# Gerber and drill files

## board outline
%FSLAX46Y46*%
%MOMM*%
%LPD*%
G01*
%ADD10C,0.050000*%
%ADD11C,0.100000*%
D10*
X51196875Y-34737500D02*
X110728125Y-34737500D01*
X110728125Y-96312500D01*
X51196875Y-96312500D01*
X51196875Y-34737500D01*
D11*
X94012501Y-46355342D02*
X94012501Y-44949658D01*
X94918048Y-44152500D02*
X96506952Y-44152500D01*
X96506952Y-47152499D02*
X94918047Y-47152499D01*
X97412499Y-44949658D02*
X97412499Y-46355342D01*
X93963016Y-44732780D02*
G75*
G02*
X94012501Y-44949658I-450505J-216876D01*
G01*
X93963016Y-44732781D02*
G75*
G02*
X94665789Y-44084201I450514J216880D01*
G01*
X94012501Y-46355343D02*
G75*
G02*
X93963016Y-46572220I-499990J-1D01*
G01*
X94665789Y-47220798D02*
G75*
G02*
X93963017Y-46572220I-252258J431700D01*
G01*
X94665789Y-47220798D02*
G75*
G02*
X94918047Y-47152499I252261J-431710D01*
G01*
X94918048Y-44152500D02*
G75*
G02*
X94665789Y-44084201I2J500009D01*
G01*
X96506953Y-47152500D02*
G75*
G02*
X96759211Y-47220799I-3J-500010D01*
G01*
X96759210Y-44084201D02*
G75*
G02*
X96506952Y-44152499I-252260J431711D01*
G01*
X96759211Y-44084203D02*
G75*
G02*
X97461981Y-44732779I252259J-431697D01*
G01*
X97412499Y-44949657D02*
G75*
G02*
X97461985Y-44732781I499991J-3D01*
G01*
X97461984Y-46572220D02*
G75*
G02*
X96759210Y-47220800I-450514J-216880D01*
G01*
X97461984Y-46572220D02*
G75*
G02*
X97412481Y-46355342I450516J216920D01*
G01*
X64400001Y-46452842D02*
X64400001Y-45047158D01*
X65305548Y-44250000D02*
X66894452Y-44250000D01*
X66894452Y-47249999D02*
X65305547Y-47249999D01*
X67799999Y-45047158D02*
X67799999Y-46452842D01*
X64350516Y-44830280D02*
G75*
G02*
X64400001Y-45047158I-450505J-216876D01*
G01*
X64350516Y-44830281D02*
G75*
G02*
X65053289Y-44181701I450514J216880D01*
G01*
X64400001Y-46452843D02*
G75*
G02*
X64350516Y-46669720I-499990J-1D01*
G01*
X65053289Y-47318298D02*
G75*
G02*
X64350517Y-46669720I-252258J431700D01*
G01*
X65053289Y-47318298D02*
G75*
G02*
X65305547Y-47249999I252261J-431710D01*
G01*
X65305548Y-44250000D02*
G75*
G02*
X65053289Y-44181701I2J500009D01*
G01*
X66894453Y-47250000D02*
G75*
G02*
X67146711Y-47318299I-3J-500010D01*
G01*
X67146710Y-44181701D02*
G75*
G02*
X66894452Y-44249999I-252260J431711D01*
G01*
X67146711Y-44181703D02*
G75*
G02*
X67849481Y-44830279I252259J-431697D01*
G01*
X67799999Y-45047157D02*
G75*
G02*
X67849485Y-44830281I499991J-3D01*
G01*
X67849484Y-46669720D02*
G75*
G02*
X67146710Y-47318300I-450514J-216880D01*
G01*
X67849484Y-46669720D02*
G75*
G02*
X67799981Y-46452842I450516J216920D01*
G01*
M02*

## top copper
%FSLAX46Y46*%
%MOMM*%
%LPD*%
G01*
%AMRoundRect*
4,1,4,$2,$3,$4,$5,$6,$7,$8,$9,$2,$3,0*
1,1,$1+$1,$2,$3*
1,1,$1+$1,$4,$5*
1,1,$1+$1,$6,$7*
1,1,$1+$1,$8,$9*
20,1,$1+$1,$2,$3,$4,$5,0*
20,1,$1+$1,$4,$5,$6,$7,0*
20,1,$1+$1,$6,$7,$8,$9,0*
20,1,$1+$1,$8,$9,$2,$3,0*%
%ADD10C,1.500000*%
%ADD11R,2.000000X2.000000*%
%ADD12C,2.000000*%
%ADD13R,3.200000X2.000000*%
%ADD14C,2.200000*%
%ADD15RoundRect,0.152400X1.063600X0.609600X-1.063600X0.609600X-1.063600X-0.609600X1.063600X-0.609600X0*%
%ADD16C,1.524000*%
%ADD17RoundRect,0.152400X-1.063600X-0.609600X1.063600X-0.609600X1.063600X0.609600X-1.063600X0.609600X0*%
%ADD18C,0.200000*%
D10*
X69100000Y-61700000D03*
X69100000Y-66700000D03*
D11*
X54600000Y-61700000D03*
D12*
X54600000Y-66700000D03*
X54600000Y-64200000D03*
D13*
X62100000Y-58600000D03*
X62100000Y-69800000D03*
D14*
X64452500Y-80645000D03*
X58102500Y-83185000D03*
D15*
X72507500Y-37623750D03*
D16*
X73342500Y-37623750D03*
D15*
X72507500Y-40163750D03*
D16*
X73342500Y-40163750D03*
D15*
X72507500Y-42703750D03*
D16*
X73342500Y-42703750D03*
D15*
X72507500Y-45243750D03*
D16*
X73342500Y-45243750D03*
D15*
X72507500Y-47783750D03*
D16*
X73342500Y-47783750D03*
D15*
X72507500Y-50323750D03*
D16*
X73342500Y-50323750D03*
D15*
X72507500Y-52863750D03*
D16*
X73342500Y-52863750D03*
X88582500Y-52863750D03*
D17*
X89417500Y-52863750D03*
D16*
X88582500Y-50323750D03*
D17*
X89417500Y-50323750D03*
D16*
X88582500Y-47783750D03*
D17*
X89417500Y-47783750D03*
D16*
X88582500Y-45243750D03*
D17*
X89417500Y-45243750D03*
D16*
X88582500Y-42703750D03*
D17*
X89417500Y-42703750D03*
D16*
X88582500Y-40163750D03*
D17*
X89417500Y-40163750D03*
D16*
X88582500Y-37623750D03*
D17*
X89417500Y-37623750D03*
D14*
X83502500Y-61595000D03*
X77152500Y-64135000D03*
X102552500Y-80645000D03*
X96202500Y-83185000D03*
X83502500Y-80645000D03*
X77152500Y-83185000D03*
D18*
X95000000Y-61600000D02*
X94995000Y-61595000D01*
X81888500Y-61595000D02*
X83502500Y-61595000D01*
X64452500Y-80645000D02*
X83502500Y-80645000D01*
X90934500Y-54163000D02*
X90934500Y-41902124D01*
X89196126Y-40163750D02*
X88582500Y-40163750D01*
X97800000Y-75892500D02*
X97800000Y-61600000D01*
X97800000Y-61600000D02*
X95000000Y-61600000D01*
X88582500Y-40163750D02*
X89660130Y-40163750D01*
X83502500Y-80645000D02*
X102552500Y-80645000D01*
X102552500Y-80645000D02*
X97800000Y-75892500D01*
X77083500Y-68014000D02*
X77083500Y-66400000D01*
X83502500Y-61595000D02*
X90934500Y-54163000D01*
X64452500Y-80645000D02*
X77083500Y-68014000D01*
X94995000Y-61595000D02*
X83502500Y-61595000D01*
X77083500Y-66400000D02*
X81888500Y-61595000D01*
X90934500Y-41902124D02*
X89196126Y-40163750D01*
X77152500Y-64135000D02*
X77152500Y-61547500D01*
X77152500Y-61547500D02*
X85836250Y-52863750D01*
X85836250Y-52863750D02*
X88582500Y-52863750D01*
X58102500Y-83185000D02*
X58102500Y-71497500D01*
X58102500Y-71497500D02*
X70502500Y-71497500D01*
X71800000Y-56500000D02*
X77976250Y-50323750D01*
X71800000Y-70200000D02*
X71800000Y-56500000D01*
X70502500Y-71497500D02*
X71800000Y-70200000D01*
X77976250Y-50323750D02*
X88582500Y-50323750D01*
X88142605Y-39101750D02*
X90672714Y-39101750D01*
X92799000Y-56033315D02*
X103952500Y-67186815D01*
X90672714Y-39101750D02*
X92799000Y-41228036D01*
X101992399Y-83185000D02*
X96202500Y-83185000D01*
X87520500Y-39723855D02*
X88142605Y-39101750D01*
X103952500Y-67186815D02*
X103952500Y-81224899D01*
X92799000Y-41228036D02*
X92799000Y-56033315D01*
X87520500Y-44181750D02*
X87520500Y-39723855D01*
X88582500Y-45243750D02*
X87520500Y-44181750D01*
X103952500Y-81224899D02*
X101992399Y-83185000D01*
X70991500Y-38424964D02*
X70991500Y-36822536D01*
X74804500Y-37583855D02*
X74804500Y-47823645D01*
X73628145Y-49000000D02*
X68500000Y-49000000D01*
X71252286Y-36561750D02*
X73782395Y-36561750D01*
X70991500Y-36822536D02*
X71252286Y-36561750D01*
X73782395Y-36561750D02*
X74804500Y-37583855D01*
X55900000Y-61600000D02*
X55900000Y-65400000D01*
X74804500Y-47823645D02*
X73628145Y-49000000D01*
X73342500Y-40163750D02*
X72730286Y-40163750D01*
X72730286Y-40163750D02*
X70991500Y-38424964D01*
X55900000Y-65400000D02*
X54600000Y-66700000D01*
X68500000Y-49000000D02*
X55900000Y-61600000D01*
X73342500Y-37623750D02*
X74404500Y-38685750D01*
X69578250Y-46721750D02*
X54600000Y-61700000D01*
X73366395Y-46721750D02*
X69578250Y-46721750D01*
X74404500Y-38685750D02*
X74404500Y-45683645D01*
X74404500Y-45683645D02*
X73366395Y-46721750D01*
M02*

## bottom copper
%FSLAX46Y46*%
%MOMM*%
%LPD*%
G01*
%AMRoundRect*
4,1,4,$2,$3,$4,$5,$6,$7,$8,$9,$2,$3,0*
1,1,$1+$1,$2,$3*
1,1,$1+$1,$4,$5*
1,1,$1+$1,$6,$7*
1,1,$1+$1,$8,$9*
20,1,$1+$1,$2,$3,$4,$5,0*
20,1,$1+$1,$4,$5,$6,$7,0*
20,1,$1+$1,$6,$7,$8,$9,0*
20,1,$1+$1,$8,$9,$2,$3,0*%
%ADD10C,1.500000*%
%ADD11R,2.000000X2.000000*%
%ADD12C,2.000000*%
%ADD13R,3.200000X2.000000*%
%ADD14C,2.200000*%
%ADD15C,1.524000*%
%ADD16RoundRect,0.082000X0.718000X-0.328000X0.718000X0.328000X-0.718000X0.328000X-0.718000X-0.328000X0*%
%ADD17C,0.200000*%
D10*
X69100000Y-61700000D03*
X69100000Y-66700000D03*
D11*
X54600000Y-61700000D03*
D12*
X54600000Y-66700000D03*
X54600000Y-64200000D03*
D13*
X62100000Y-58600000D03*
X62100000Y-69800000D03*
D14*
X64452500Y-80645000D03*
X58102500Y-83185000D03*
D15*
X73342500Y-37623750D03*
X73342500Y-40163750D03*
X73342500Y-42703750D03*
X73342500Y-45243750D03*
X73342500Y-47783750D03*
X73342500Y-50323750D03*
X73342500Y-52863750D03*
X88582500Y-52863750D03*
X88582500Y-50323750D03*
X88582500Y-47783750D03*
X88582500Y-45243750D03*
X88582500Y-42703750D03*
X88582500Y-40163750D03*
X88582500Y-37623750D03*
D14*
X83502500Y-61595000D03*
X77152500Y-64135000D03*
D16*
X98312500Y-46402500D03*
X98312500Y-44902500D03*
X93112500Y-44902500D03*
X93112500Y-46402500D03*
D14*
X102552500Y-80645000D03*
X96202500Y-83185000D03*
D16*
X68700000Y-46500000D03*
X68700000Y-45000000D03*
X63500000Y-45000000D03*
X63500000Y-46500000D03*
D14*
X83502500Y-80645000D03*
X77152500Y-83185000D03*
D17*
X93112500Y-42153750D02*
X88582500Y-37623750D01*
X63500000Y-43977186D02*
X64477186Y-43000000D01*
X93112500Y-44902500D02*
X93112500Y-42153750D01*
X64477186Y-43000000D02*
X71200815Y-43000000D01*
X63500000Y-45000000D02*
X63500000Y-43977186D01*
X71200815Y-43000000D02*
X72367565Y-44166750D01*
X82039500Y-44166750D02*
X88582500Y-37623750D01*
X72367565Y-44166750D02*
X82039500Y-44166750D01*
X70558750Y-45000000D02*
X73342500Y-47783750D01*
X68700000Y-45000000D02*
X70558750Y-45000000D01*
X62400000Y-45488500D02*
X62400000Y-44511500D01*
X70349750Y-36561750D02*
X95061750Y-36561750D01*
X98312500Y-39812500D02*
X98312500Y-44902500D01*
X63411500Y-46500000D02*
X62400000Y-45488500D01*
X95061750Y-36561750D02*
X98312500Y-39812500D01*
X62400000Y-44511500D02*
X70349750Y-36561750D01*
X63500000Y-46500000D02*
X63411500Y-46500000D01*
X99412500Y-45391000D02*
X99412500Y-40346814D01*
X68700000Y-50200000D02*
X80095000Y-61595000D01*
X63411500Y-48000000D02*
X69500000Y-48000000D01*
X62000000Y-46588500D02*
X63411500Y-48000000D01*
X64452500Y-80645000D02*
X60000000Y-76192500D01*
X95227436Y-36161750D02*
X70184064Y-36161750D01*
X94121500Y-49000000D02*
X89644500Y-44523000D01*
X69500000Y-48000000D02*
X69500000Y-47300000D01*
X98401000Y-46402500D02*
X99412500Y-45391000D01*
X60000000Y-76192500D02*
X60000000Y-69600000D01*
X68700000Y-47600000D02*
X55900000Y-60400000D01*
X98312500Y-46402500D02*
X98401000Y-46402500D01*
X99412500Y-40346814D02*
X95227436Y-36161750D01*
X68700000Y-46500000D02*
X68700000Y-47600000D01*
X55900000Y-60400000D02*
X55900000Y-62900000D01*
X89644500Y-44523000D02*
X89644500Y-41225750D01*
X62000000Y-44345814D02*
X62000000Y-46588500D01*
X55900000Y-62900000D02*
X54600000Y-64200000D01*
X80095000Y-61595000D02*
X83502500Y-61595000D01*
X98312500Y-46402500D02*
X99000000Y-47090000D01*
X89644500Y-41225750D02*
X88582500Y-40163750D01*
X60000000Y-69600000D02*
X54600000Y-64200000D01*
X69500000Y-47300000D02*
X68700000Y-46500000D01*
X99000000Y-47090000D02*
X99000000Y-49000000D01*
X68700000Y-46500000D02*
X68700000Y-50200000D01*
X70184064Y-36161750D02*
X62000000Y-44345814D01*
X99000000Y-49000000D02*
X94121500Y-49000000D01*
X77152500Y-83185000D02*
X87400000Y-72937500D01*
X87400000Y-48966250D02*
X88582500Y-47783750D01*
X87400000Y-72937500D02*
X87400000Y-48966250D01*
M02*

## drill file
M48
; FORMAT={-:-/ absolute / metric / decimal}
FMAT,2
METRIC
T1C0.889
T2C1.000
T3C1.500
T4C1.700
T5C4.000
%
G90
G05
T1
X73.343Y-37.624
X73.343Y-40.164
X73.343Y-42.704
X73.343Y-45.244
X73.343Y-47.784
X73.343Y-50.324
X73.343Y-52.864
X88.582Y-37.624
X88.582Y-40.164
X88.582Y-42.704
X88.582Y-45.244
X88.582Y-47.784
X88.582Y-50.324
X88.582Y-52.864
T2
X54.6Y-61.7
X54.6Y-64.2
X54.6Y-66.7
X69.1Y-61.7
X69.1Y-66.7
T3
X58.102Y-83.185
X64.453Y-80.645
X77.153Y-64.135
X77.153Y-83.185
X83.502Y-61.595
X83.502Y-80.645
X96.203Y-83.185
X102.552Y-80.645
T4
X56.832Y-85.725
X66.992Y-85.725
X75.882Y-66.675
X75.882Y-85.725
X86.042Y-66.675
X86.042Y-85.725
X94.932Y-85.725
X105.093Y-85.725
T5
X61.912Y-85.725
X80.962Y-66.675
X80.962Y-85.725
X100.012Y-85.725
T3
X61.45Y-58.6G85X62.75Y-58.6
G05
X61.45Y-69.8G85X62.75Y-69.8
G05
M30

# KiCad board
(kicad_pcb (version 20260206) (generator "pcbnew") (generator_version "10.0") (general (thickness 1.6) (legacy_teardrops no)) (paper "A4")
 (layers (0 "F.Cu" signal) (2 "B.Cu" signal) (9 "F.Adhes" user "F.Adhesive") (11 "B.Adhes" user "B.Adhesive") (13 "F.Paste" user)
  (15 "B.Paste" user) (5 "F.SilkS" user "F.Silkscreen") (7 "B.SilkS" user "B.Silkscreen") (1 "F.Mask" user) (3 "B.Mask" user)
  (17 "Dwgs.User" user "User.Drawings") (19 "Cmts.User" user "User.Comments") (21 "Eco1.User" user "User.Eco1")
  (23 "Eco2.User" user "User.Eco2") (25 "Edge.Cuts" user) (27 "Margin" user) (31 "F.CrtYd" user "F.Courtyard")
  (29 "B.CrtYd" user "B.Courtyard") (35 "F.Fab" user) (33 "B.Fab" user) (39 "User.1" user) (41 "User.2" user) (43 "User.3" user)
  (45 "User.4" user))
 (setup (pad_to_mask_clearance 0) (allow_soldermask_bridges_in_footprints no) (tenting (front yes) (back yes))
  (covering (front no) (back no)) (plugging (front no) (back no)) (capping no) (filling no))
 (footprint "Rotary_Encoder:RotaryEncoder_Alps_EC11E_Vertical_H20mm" (layer "F.Cu") (at 54.6 61.7)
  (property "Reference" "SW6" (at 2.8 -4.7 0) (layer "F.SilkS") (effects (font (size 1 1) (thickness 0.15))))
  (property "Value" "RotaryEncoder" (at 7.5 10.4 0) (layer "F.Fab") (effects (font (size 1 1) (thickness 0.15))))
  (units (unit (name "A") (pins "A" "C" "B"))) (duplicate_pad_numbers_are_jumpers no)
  (pad "" thru_hole circle (at 14.5 0) (size 1.5 1.5) (drill 1) (layers "*.Cu" "*.Mask") (remove_unused_layers no))
  (pad "" thru_hole circle (at 14.5 5) (size 1.5 1.5) (drill 1) (layers "*.Cu" "*.Mask") (remove_unused_layers no))
  (pad "A" thru_hole rect (at 0 0) (size 2 2) (drill 1) (layers "*.Cu" "*.Mask") (remove_unused_layers no)
   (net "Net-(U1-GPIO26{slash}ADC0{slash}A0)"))
  (pad "B" thru_hole circle (at 0 5) (size 2 2) (drill 1) (layers "*.Cu" "*.Mask") (remove_unused_layers no)
   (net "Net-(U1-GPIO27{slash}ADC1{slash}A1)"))
  (pad "C" thru_hole circle (at 0 2.5) (size 2 2) (drill 1) (layers "*.Cu" "*.Mask") (remove_unused_layers no) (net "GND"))
  (pad "MP" thru_hole rect (at 7.5 -3.1) (size 3.2 2) (drill oval 2.8 1.5) (layers "*.Cu" "*.Mask") (remove_unused_layers no))
  (pad "MP" thru_hole rect (at 7.5 8.1) (size 3.2 2) (drill oval 2.8 1.5) (layers "*.Cu" "*.Mask") (remove_unused_layers no)))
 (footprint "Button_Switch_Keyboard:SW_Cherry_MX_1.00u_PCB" (layer "F.Cu") (at 64.4525 80.645)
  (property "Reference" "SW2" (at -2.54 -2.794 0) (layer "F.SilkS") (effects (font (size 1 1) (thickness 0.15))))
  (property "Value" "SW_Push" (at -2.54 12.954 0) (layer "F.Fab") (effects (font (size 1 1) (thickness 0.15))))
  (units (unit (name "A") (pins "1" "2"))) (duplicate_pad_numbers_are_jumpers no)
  (pad "" np_thru_hole circle (at -7.62 5.08) (size 1.7 1.7) (drill 1.7) (layers "*.Cu" "*.Mask"))
  (pad "" np_thru_hole circle (at -2.54 5.08) (size 4 4) (drill 4) (layers "*.Cu" "*.Mask"))
  (pad "" np_thru_hole circle (at 2.54 5.08) (size 1.7 1.7) (drill 1.7) (layers "*.Cu" "*.Mask"))
  (pad "1" thru_hole circle (at 0 0) (size 2.2 2.2) (drill 1.5) (layers "*.Cu" "*.Mask") (remove_unused_layers no) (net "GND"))
  (pad "2" thru_hole circle (at -6.35 2.54) (size 2.2 2.2) (drill 1.5) (layers "*.Cu" "*.Mask") (remove_unused_layers no)
   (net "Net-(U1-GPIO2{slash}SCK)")))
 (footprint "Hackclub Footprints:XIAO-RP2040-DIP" (layer "F.Cu") (at 80.9625 45.24375)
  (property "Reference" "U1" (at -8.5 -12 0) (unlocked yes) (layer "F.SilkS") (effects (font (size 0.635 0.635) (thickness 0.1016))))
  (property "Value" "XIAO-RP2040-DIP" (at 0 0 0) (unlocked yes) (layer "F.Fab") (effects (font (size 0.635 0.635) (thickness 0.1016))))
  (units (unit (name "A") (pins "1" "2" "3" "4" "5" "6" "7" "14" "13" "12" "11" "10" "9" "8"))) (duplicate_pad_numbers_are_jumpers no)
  (pad "1" smd roundrect (at -8.455 -7.62 180) (size 2.432 1.524) (layers "F.Cu" "F.Mask") (roundrect_rratio 0.1)
   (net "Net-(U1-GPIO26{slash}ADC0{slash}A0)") (thermal_bridge_angle 45))
  (pad "1" thru_hole circle (at -7.62 -7.62 180) (size 1.524 1.524) (drill 0.889) (layers "*.Cu" "*.Mask") (remove_unused_layers no)
   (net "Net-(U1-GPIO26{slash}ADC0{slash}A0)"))
  (pad "2" smd roundrect (at -8.455 -5.08 180) (size 2.432 1.524) (layers "F.Cu" "F.Mask") (roundrect_rratio 0.1)
   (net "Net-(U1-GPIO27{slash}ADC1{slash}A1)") (thermal_bridge_angle 45))
  (pad "2" thru_hole circle (at -7.62 -5.08 180) (size 1.524 1.524) (drill 0.889) (layers "*.Cu" "*.Mask") (remove_unused_layers no)
   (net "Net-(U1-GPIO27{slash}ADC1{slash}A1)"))
  (pad "3" smd roundrect (at -8.455 -2.54 180) (size 2.432 1.524) (layers "F.Cu" "F.Mask") (roundrect_rratio 0.1)
   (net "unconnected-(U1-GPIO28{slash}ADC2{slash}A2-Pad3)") (thermal_bridge_angle 45))
  (pad "3" thru_hole circle (at -7.62 -2.54 180) (size 1.524 1.524) (drill 0.889) (layers "*.Cu" "*.Mask") (remove_unused_layers no)
   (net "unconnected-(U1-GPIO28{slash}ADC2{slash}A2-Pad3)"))
  (pad "4" smd roundrect (at -8.455 0 180) (size 2.432 1.524) (layers "F.Cu" "F.Mask") (roundrect_rratio 0.1)
   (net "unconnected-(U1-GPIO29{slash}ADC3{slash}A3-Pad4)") (thermal_bridge_angle 45))
  (pad "4" thru_hole circle (at -7.62 0 180) (size 1.524 1.524) (drill 0.889) (layers "*.Cu" "*.Mask") (remove_unused_layers no)
   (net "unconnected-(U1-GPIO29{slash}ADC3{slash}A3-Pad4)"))
  (pad "5" smd roundrect (at -8.455 2.54 180) (size 2.432 1.524) (layers "F.Cu" "F.Mask") (roundrect_rratio 0.1) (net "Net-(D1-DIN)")
   (thermal_bridge_angle 45))
  (pad "5" thru_hole circle (at -7.62 2.54 180) (size 1.524 1.524) (drill 0.889) (layers "*.Cu" "*.Mask") (remove_unused_layers no)
   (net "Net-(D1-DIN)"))
  (pad "6" smd roundrect (at -8.455 5.08 180) (size 2.432 1.524) (layers "F.Cu" "F.Mask") (roundrect_rratio 0.1)
   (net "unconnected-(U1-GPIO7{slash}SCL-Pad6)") (thermal_bridge_angle 45))
  (pad "6" thru_hole circle (at -7.62 5.08 180) (size 1.524 1.524) (drill 0.889) (layers "*.Cu" "*.Mask") (remove_unused_layers no)
   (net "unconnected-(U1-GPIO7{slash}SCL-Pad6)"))
  (pad "7" smd roundrect (at -8.455 7.62 180) (size 2.432 1.524) (layers "F.Cu" "F.Mask") (roundrect_rratio 0.1)
   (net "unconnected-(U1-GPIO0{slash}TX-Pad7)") (thermal_bridge_angle 45))
  (pad "7" thru_hole circle (at -7.62 7.62 180) (size 1.524 1.524) (drill 0.889) (layers "*.Cu" "*.Mask") (remove_unused_layers no)
   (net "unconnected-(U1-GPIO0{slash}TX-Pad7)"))
  (pad "8" thru_hole circle (at 7.62 7.62) (size 1.524 1.524) (drill 0.889) (layers "*.Cu" "*.Mask") (remove_unused_layers no)
   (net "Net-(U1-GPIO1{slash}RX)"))
  (pad "8" smd roundrect (at 8.455 7.62) (size 2.432 1.524) (layers "F.Cu" "F.Mask") (roundrect_rratio 0.1) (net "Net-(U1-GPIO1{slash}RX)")
   (thermal_bridge_angle 45))
  (pad "9" thru_hole circle (at 7.62 5.08) (size 1.524 1.524) (drill 0.889) (layers "*.Cu" "*.Mask") (remove_unused_layers no)
   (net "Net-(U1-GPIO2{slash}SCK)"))
  (pad "9" smd roundrect (at 8.455 5.08) (size 2.432 1.524) (layers "F.Cu" "F.Mask") (roundrect_rratio 0.1) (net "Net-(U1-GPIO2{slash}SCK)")
   (thermal_bridge_angle 45))
  (pad "10" thru_hole circle (at 7.62 2.54) (size 1.524 1.524) (drill 0.889) (layers "*.Cu" "*.Mask") (remove_unused_layers no)
   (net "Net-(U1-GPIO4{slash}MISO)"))
  (pad "10" smd roundrect (at 8.455 2.54) (size 2.432 1.524) (layers "F.Cu" "F.Mask") (roundrect_rratio 0.1)
   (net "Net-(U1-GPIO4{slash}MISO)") (thermal_bridge_angle 45))
  (pad "11" thru_hole circle (at 7.62 0) (size 1.524 1.524) (drill 0.889) (layers "*.Cu" "*.Mask") (remove_unused_layers no)
   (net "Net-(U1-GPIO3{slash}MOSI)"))
  (pad "11" smd roundrect (at 8.455 0) (size 2.432 1.524) (layers "F.Cu" "F.Mask") (roundrect_rratio 0.1) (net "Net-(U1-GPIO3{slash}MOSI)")
   (thermal_bridge_angle 45))
  (pad "12" thru_hole circle (at 7.62 -2.54) (size 1.524 1.524) (drill 0.889) (layers "*.Cu" "*.Mask") (remove_unused_layers no)
   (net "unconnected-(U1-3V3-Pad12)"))
  (pad "12" smd roundrect (at 8.455 -2.54) (size 2.432 1.524) (layers "F.Cu" "F.Mask") (roundrect_rratio 0.1)
   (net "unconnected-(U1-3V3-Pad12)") (thermal_bridge_angle 45))
  (pad "13" thru_hole circle (at 7.62 -5.08) (size 1.524 1.524) (drill 0.889) (layers "*.Cu" "*.Mask") (remove_unused_layers no) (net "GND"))
  (pad "13" smd roundrect (at 8.455 -5.08) (size 2.432 1.524) (layers "F.Cu" "F.Mask") (roundrect_rratio 0.1) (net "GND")
   (thermal_bridge_angle 45))
  (pad "14" thru_hole circle (at 7.62 -7.62) (size 1.524 1.524) (drill 0.889) (layers "*.Cu" "*.Mask") (remove_unused_layers no) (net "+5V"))
  (pad "14" smd roundrect (at 8.455 -7.62) (size 2.432 1.524) (layers "F.Cu" "F.Mask") (roundrect_rratio 0.1) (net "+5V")
   (thermal_bridge_angle 45)))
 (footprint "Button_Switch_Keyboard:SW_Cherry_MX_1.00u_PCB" (layer "F.Cu") (at 83.5025 61.595)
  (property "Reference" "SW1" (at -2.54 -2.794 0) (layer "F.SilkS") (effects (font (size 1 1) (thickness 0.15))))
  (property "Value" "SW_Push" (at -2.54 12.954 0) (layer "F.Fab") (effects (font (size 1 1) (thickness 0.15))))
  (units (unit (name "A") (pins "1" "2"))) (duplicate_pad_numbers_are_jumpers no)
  (pad "" np_thru_hole circle (at -7.62 5.08) (size 1.7 1.7) (drill 1.7) (layers "*.Cu" "*.Mask"))
  (pad "" np_thru_hole circle (at -2.54 5.08) (size 4 4) (drill 4) (layers "*.Cu" "*.Mask"))
  (pad "" np_thru_hole circle (at 2.54 5.08) (size 1.7 1.7) (drill 1.7) (layers "*.Cu" "*.Mask"))
  (pad "1" thru_hole circle (at 0 0) (size 2.2 2.2) (drill 1.5) (layers "*.Cu" "*.Mask") (remove_unused_layers no) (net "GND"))
  (pad "2" thru_hole circle (at -6.35 2.54) (size 2.2 2.2) (drill 1.5) (layers "*.Cu" "*.Mask") (remove_unused_layers no)
   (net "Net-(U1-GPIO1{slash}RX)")))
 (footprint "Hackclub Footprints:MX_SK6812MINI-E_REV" (layer "F.Cu") (at 95.7125 40.5725)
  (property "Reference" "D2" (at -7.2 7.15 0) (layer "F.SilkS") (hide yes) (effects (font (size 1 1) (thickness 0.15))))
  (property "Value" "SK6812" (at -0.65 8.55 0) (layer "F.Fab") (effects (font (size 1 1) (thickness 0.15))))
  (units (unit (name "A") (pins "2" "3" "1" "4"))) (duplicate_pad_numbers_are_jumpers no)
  (fp_line (start -1.699999 5.782842) (end -1.699999 4.377158) (stroke (width 0.1) (type solid)) (layer "Edge.Cuts"))
  (fp_line (start -0.794452 3.58) (end 0.794452 3.58) (stroke (width 0.1) (type solid)) (layer "Edge.Cuts"))
  (fp_line (start 0.794452 6.579999) (end -0.794453 6.579999) (stroke (width 0.1) (type solid)) (layer "Edge.Cuts"))
  (fp_line (start 1.699999 4.377158) (end 1.699999 5.782842) (stroke (width 0.1) (type solid)) (layer "Edge.Cuts"))
  (fp_arc (start -1.749484 4.16028) (mid -1.712527 4.265932) (end -1.699999 4.377158) (stroke (width 0.1) (type solid)) (layer "Edge.Cuts"))
  (fp_arc (start -1.749484 4.160281) (mid -1.638072 3.575965) (end -1.046711 3.511701) (stroke (width 0.1) (type solid)) (layer "Edge.Cuts"))
  (fp_arc (start -1.699999 5.782843) (mid -1.712527 5.894068) (end -1.749484 5.99972) (stroke (width 0.1) (type solid)) (layer "Edge.Cuts"))
  (fp_arc (start -1.046711 6.648298) (mid -1.638071 6.584034) (end -1.749484 5.99972) (stroke (width 0.1) (type solid)) (layer "Edge.Cuts"))
  (fp_arc (start -1.046711 6.648298) (mid -0.925123 6.597376) (end -0.794453 6.579999) (stroke (width 0.1) (type solid)) (layer "Edge.Cuts"))
  (fp_arc (start -0.794452 3.58) (mid -0.925123 3.562623) (end -1.046711 3.511701) (stroke (width 0.1) (type solid)) (layer "Edge.Cuts"))
  (fp_arc (start 0.794453 6.58) (mid 0.925123 6.597377) (end 1.046711 6.648299) (stroke (width 0.1) (type solid)) (layer "Edge.Cuts"))
  (fp_arc (start 1.04671 3.511701) (mid 0.925122 3.562623) (end 0.794452 3.58) (stroke (width 0.1) (type solid)) (layer "Edge.Cuts"))
  (fp_arc (start 1.046711 3.511703) (mid 1.63807 3.575966) (end 1.749484 4.16028) (stroke (width 0.1) (type solid)) (layer "Edge.Cuts"))
  (fp_arc (start 1.699999 4.377157) (mid 1.712527 4.265932) (end 1.749484 4.16028) (stroke (width 0.1) (type solid)) (layer "Edge.Cuts"))
  (fp_arc (start 1.749484 5.99972) (mid 1.638071 6.584035) (end 1.046711 6.648299) (stroke (width 0.1) (type solid)) (layer "Edge.Cuts"))
  (fp_arc (start 1.749484 5.99972) (mid 1.712527 5.894068) (end 1.699999 5.782842) (stroke (width 0.1) (type solid)) (layer "Edge.Cuts"))
  (pad "1" smd roundrect (at 2.6 5.83 90) (size 0.82 1.6) (layers "B.Cu" "B.Mask" "B.Paste") (roundrect_rratio 0.1) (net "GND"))
  (pad "2" smd roundrect (at 2.6 4.33 90) (size 0.82 1.6) (layers "B.Cu" "B.Mask" "B.Paste") (roundrect_rratio 0.1) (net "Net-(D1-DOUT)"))
  (pad "3" smd roundrect (at -2.6 4.33 90) (size 0.82 1.6) (layers "B.Cu" "B.Mask" "B.Paste") (roundrect_rratio 0.1) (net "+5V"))
  (pad "4" smd roundrect (at -2.6 5.83 90) (size 0.82 1.6) (layers "B.Cu" "B.Mask" "B.Paste") (roundrect_rratio 0.1)
   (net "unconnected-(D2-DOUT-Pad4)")))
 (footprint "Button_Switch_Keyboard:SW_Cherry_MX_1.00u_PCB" (layer "F.Cu") (at 102.5525 80.645)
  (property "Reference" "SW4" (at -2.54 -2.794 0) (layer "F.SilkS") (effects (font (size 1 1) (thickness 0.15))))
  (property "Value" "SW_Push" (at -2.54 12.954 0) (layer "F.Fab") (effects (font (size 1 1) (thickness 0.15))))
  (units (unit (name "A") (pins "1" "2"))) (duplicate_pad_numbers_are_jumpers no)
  (pad "" np_thru_hole circle (at -7.62 5.08) (size 1.7 1.7) (drill 1.7) (layers "*.Cu" "*.Mask"))
  (pad "" np_thru_hole circle (at -2.54 5.08) (size 4 4) (drill 4) (layers "*.Cu" "*.Mask"))
  (pad "" np_thru_hole circle (at 2.54 5.08) (size 1.7 1.7) (drill 1.7) (layers "*.Cu" "*.Mask"))
  (pad "1" thru_hole circle (at 0 0) (size 2.2 2.2) (drill 1.5) (layers "*.Cu" "*.Mask") (remove_unused_layers no) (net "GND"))
  (pad "2" thru_hole circle (at -6.35 2.54) (size 2.2 2.2) (drill 1.5) (layers "*.Cu" "*.Mask") (remove_unused_layers no)
   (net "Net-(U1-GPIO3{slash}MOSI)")))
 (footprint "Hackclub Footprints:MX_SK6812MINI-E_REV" (layer "F.Cu") (at 66.1 40.67)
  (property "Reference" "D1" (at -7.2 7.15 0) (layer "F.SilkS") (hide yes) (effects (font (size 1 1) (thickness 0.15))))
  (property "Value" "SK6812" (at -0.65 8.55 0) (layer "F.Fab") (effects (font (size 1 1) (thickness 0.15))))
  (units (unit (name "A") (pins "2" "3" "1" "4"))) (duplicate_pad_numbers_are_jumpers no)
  (fp_line (start -1.699999 5.782842) (end -1.699999 4.377158) (stroke (width 0.1) (type solid)) (layer "Edge.Cuts"))
  (fp_line (start -0.794452 3.58) (end 0.794452 3.58) (stroke (width 0.1) (type solid)) (layer "Edge.Cuts"))
  (fp_line (start 0.794452 6.579999) (end -0.794453 6.579999) (stroke (width 0.1) (type solid)) (layer "Edge.Cuts"))
  (fp_line (start 1.699999 4.377158) (end 1.699999 5.782842) (stroke (width 0.1) (type solid)) (layer "Edge.Cuts"))
  (fp_arc (start -1.749484 4.16028) (mid -1.712527 4.265932) (end -1.699999 4.377158) (stroke (width 0.1) (type solid)) (layer "Edge.Cuts"))
  (fp_arc (start -1.749484 4.160281) (mid -1.638072 3.575965) (end -1.046711 3.511701) (stroke (width 0.1) (type solid)) (layer "Edge.Cuts"))
  (fp_arc (start -1.699999 5.782843) (mid -1.712527 5.894068) (end -1.749484 5.99972) (stroke (width 0.1) (type solid)) (layer "Edge.Cuts"))
  (fp_arc (start -1.046711 6.648298) (mid -1.638071 6.584034) (end -1.749484 5.99972) (stroke (width 0.1) (type solid)) (layer "Edge.Cuts"))
  (fp_arc (start -1.046711 6.648298) (mid -0.925123 6.597376) (end -0.794453 6.579999) (stroke (width 0.1) (type solid)) (layer "Edge.Cuts"))
  (fp_arc (start -0.794452 3.58) (mid -0.925123 3.562623) (end -1.046711 3.511701) (stroke (width 0.1) (type solid)) (layer "Edge.Cuts"))
  (fp_arc (start 0.794453 6.58) (mid 0.925123 6.597377) (end 1.046711 6.648299) (stroke (width 0.1) (type solid)) (layer "Edge.Cuts"))
  (fp_arc (start 1.04671 3.511701) (mid 0.925122 3.562623) (end 0.794452 3.58) (stroke (width 0.1) (type solid)) (layer "Edge.Cuts"))
  (fp_arc (start 1.046711 3.511703) (mid 1.63807 3.575966) (end 1.749484 4.16028) (stroke (width 0.1) (type solid)) (layer "Edge.Cuts"))
  (fp_arc (start 1.699999 4.377157) (mid 1.712527 4.265932) (end 1.749484 4.16028) (stroke (width 0.1) (type solid)) (layer "Edge.Cuts"))
  (fp_arc (start 1.749484 5.99972) (mid 1.638071 6.584035) (end 1.046711 6.648299) (stroke (width 0.1) (type solid)) (layer "Edge.Cuts"))
  (fp_arc (start 1.749484 5.99972) (mid 1.712527 5.894068) (end 1.699999 5.782842) (stroke (width 0.1) (type solid)) (layer "Edge.Cuts"))
  (pad "1" smd roundrect (at 2.6 5.83 90) (size 0.82 1.6) (layers "B.Cu" "B.Mask" "B.Paste") (roundrect_rratio 0.1) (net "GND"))
  (pad "2" smd roundrect (at 2.6 4.33 90) (size 0.82 1.6) (layers "B.Cu" "B.Mask" "B.Paste") (roundrect_rratio 0.1) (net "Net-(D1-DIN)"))
  (pad "3" smd roundrect (at -2.6 4.33 90) (size 0.82 1.6) (layers "B.Cu" "B.Mask" "B.Paste") (roundrect_rratio 0.1) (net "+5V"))
  (pad "4" smd roundrect (at -2.6 5.83 90) (size 0.82 1.6) (layers "B.Cu" "B.Mask" "B.Paste") (roundrect_rratio 0.1) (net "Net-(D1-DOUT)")))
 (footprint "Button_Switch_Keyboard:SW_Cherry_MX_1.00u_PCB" (layer "F.Cu") (at 83.5025 80.645)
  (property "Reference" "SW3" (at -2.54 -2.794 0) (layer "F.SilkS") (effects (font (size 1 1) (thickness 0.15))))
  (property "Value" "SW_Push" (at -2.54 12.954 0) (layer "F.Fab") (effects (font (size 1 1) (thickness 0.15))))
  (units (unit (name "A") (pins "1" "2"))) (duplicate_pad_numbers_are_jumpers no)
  (pad "" np_thru_hole circle (at -7.62 5.08) (size 1.7 1.7) (drill 1.7) (layers "*.Cu" "*.Mask"))
  (pad "" np_thru_hole circle (at -2.54 5.08) (size 4 4) (drill 4) (layers "*.Cu" "*.Mask"))
  (pad "" np_thru_hole circle (at 2.54 5.08) (size 1.7 1.7) (drill 1.7) (layers "*.Cu" "*.Mask"))
  (pad "1" thru_hole circle (at 0 0) (size 2.2 2.2) (drill 1.5) (layers "*.Cu" "*.Mask") (remove_unused_layers no) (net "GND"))
  (pad "2" thru_hole circle (at -6.35 2.54) (size 2.2 2.2) (drill 1.5) (layers "*.Cu" "*.Mask") (remove_unused_layers no)
   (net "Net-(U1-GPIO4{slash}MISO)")))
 (gr_rect (start 51.196875 34.7375) (end 110.728125 96.3125) (stroke (width 0.05) (type solid)) (fill no) (layer "Edge.Cuts"))
 (segment (start 93.1125 42.15375) (end 88.5825 37.62375) (width 0.2) (layer "B.Cu") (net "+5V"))
 (segment (start 63.5 43.977186) (end 64.477186 43) (width 0.2) (layer "B.Cu") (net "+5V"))
 (segment (start 93.1125 44.9025) (end 93.1125 42.15375) (width 0.2) (layer "B.Cu") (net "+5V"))
 (segment (start 64.477186 43) (end 71.200815 43) (width 0.2) (layer "B.Cu") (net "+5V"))
 (segment (start 63.5 45) (end 63.5 43.977186) (width 0.2) (layer "B.Cu") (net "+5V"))
 (segment (start 71.200815 43) (end 72.367565 44.16675) (width 0.2) (layer "B.Cu") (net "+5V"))
 (segment (start 82.0395 44.16675) (end 88.5825 37.62375) (width 0.2) (layer "B.Cu") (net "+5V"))
 (segment (start 72.367565 44.16675) (end 82.0395 44.16675) (width 0.2) (layer "B.Cu") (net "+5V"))
 (segment (start 70.55875 45) (end 73.3425 47.78375) (width 0.2) (layer "B.Cu") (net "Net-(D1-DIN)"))
 (segment (start 68.7 45) (end 70.55875 45) (width 0.2) (layer "B.Cu") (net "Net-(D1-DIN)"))
 (segment (start 62.4 45.4885) (end 62.4 44.5115) (width 0.2) (layer "B.Cu") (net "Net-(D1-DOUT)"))
 (segment (start 70.34975 36.56175) (end 95.06175 36.56175) (width 0.2) (layer "B.Cu") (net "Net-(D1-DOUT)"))
 (segment (start 98.3125 39.8125) (end 98.3125 44.9025) (width 0.2) (layer "B.Cu") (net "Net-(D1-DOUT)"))
 (segment (start 63.4115 46.5) (end 62.4 45.4885) (width 0.2) (layer "B.Cu") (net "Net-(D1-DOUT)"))
 (segment (start 95.06175 36.56175) (end 98.3125 39.8125) (width 0.2) (layer "B.Cu") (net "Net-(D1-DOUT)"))
 (segment (start 62.4 44.5115) (end 70.34975 36.56175) (width 0.2) (layer "B.Cu") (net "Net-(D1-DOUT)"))
 (segment (start 63.5 46.5) (end 63.4115 46.5) (width 0.2) (layer "B.Cu") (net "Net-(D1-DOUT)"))
 (segment (start 95 61.6) (end 94.995 61.595) (width 0.2) (layer "F.Cu") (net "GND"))
 (segment (start 81.8885 61.595) (end 83.5025 61.595) (width 0.2) (layer "F.Cu") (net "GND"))
 (segment (start 64.4525 80.645) (end 83.5025 80.645) (width 0.2) (layer "F.Cu") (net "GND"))
 (segment (start 90.9345 54.163) (end 90.9345 41.902124) (width 0.2) (layer "F.Cu") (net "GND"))
 (segment (start 89.196126 40.16375) (end 88.5825 40.16375) (width 0.2) (layer "F.Cu") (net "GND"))
 (segment (start 97.8 75.8925) (end 97.8 61.6) (width 0.2) (layer "F.Cu") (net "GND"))
 (segment (start 97.8 61.6) (end 95 61.6) (width 0.2) (layer "F.Cu") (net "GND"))
 (segment (start 88.5825 40.16375) (end 89.66013 40.16375) (width 0.2) (layer "F.Cu") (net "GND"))
 (segment (start 83.5025 80.645) (end 102.5525 80.645) (width 0.2) (layer "F.Cu") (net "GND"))
 (segment (start 102.5525 80.645) (end 97.8 75.8925) (width 0.2) (layer "F.Cu") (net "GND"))
 (segment (start 77.0835 68.014) (end 77.0835 66.4) (width 0.2) (layer "F.Cu") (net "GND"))
 (segment (start 83.5025 61.595) (end 90.9345 54.163) (width 0.2) (layer "F.Cu") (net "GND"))
 (segment (start 64.4525 80.645) (end 77.0835 68.014) (width 0.2) (layer "F.Cu") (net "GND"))
 (segment (start 94.995 61.595) (end 83.5025 61.595) (width 0.2) (layer "F.Cu") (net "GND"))
 (segment (start 77.0835 66.4) (end 81.8885 61.595) (width 0.2) (layer "F.Cu") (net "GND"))
 (segment (start 90.9345 41.902124) (end 89.196126 40.16375) (width 0.2) (layer "F.Cu") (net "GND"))
 (segment (start 99.4125 45.391) (end 99.4125 40.346814) (width 0.2) (layer "B.Cu") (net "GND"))
 (segment (start 68.7 50.2) (end 80.095 61.595) (width 0.2) (layer "B.Cu") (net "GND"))
 (segment (start 63.4115 48) (end 69.5 48) (width 0.2) (layer "B.Cu") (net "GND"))
 (segment (start 62 46.5885) (end 63.4115 48) (width 0.2) (layer "B.Cu") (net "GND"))
 (segment (start 64.4525 80.645) (end 60 76.1925) (width 0.2) (layer "B.Cu") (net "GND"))
 (segment (start 95.227436 36.16175) (end 70.184064 36.16175) (width 0.2) (layer "B.Cu") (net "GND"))
 (segment (start 94.1215 49) (end 89.6445 44.523) (width 0.2) (layer "B.Cu") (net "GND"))
 (segment (start 69.5 48) (end 69.5 47.3) (width 0.2) (layer "B.Cu") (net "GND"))
 (segment (start 98.401 46.4025) (end 99.4125 45.391) (width 0.2) (layer "B.Cu") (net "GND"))
 (segment (start 60 76.1925) (end 60 69.6) (width 0.2) (layer "B.Cu") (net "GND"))
 (segment (start 68.7 47.6) (end 55.9 60.4) (width 0.2) (layer "B.Cu") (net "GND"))
 (segment (start 98.3125 46.4025) (end 98.401 46.4025) (width 0.2) (layer "B.Cu") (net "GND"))
 (segment (start 99.4125 40.346814) (end 95.227436 36.16175) (width 0.2) (layer "B.Cu") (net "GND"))
 (segment (start 68.7 46.5) (end 68.7 47.6) (width 0.2) (layer "B.Cu") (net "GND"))
 (segment (start 55.9 60.4) (end 55.9 62.9) (width 0.2) (layer "B.Cu") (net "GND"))
 (segment (start 89.6445 44.523) (end 89.6445 41.22575) (width 0.2) (layer "B.Cu") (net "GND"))
 (segment (start 62 44.345814) (end 62 46.5885) (width 0.2) (layer "B.Cu") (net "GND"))
 (segment (start 55.9 62.9) (end 54.6 64.2) (width 0.2) (layer "B.Cu") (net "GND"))
 (segment (start 80.095 61.595) (end 83.5025 61.595) (width 0.2) (layer "B.Cu") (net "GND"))
 (segment (start 98.3125 46.4025) (end 99 47.09) (width 0.2) (layer "B.Cu") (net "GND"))
 (segment (start 89.6445 41.22575) (end 88.5825 40.16375) (width 0.2) (layer "B.Cu") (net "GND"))
 (segment (start 60 69.6) (end 54.6 64.2) (width 0.2) (layer "B.Cu") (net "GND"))
 (segment (start 69.5 47.3) (end 68.7 46.5) (width 0.2) (layer "B.Cu") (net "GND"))
 (segment (start 99 47.09) (end 99 49) (width 0.2) (layer "B.Cu") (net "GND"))
 (segment (start 68.7 46.5) (end 68.7 50.2) (width 0.2) (layer "B.Cu") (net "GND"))
 (segment (start 70.184064 36.16175) (end 62 44.345814) (width 0.2) (layer "B.Cu") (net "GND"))
 (segment (start 99 49) (end 94.1215 49) (width 0.2) (layer "B.Cu") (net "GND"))
 (segment (start 77.1525 64.135) (end 77.1525 61.5475) (width 0.2) (layer "F.Cu") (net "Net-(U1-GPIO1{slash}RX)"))
 (segment (start 77.1525 61.5475) (end 85.83625 52.86375) (width 0.2) (layer "F.Cu") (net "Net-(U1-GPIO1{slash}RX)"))
 (segment (start 85.83625 52.86375) (end 88.5825 52.86375) (width 0.2) (layer "F.Cu") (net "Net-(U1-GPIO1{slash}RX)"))
 (segment (start 58.1025 83.185) (end 58.1025 71.4975) (width 0.2) (layer "F.Cu") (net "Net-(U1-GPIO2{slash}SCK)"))
 (segment (start 58.1025 71.4975) (end 70.5025 71.4975) (width 0.2) (layer "F.Cu") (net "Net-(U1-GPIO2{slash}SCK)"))
 (segment (start 71.8 56.5) (end 77.97625 50.32375) (width 0.2) (layer "F.Cu") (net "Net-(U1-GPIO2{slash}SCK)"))
 (segment (start 71.8 70.2) (end 71.8 56.5) (width 0.2) (layer "F.Cu") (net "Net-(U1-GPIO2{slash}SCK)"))
 (segment (start 70.5025 71.4975) (end 71.8 70.2) (width 0.2) (layer "F.Cu") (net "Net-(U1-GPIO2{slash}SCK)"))
 (segment (start 77.97625 50.32375) (end 88.5825 50.32375) (width 0.2) (layer "F.Cu") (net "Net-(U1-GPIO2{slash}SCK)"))
 (segment (start 77.1525 83.185) (end 87.4 72.9375) (width 0.2) (layer "B.Cu") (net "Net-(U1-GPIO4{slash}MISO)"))
 (segment (start 87.4 48.96625) (end 88.5825 47.78375) (width 0.2) (layer "B.Cu") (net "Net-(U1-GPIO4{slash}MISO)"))
 (segment (start 87.4 72.9375) (end 87.4 48.96625) (width 0.2) (layer "B.Cu") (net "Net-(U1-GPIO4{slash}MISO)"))
 (segment (start 88.142605 39.10175) (end 90.672714 39.10175) (width 0.2) (layer "F.Cu") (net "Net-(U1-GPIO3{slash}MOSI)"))
 (segment (start 92.799 56.033315) (end 103.9525 67.186815) (width 0.2) (layer "F.Cu") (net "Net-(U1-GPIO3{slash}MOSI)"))
 (segment (start 90.672714 39.10175) (end 92.799 41.228036) (width 0.2) (layer "F.Cu") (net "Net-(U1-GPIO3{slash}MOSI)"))
 (segment (start 101.992399 83.185) (end 96.2025 83.185) (width 0.2) (layer "F.Cu") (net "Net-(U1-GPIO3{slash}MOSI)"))
 (segment (start 87.5205 39.723855) (end 88.142605 39.10175) (width 0.2) (layer "F.Cu") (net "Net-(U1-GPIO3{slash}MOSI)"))
 (segment (start 103.9525 67.186815) (end 103.9525 81.224899) (width 0.2) (layer "F.Cu") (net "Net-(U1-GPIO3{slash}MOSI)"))
 (segment (start 92.799 41.228036) (end 92.799 56.033315) (width 0.2) (layer "F.Cu") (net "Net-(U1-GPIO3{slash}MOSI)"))
 (segment (start 87.5205 44.18175) (end 87.5205 39.723855) (width 0.2) (layer "F.Cu") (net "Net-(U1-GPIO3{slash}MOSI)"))
 (segment (start 88.5825 45.24375) (end 87.5205 44.18175) (width 0.2) (layer "F.Cu") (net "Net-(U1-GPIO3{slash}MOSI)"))
 (segment (start 103.9525 81.224899) (end 101.992399 83.185) (width 0.2) (layer "F.Cu") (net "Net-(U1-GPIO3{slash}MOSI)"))
 (segment (start 70.9915 38.424964) (end 70.9915 36.822536) (width 0.2) (layer "F.Cu") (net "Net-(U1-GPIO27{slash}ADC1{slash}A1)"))
 (segment (start 74.8045 37.583855) (end 74.8045 47.823645) (width 0.2) (layer "F.Cu") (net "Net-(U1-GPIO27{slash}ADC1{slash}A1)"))
 (segment (start 73.628145 49) (end 68.5 49) (width 0.2) (layer "F.Cu") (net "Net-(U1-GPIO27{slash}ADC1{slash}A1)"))
 (segment (start 71.252286 36.56175) (end 73.782395 36.56175) (width 0.2) (layer "F.Cu") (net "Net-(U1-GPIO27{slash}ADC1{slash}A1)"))
 (segment (start 70.9915 36.822536) (end 71.252286 36.56175) (width 0.2) (layer "F.Cu") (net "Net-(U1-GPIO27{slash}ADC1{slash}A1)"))
 (segment (start 73.782395 36.56175) (end 74.8045 37.583855) (width 0.2) (layer "F.Cu") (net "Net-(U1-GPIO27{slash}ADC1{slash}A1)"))
 (segment (start 55.9 61.6) (end 55.9 65.4) (width 0.2) (layer "F.Cu") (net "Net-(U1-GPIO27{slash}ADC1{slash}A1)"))
 (segment (start 74.8045 47.823645) (end 73.628145 49) (width 0.2) (layer "F.Cu") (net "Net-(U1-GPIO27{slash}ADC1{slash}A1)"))
 (segment (start 73.3425 40.16375) (end 72.730286 40.16375) (width 0.2) (layer "F.Cu") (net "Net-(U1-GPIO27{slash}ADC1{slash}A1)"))
 (segment (start 72.730286 40.16375) (end 70.9915 38.424964) (width 0.2) (layer "F.Cu") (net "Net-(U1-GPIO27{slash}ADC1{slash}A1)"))
 (segment (start 55.9 65.4) (end 54.6 66.7) (width 0.2) (layer "F.Cu") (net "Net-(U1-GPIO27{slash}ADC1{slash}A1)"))
 (segment (start 68.5 49) (end 55.9 61.6) (width 0.2) (layer "F.Cu") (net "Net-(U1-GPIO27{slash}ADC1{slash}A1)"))
 (segment (start 73.3425 37.62375) (end 74.4045 38.68575) (width 0.2) (layer "F.Cu") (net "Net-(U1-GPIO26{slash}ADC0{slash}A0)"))
 (segment (start 69.57825 46.72175) (end 54.6 61.7) (width 0.2) (layer "F.Cu") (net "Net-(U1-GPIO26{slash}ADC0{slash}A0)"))
 (segment (start 73.366395 46.72175) (end 69.57825 46.72175) (width 0.2) (layer "F.Cu") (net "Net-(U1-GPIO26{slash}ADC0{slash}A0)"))
 (segment (start 74.4045 38.68575) (end 74.4045 45.683645) (width 0.2) (layer "F.Cu") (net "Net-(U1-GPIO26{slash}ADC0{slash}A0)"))
 (segment (start 74.4045 45.683645) (end 73.366395 46.72175) (width 0.2) (layer "F.Cu") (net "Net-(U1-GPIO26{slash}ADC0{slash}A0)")))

